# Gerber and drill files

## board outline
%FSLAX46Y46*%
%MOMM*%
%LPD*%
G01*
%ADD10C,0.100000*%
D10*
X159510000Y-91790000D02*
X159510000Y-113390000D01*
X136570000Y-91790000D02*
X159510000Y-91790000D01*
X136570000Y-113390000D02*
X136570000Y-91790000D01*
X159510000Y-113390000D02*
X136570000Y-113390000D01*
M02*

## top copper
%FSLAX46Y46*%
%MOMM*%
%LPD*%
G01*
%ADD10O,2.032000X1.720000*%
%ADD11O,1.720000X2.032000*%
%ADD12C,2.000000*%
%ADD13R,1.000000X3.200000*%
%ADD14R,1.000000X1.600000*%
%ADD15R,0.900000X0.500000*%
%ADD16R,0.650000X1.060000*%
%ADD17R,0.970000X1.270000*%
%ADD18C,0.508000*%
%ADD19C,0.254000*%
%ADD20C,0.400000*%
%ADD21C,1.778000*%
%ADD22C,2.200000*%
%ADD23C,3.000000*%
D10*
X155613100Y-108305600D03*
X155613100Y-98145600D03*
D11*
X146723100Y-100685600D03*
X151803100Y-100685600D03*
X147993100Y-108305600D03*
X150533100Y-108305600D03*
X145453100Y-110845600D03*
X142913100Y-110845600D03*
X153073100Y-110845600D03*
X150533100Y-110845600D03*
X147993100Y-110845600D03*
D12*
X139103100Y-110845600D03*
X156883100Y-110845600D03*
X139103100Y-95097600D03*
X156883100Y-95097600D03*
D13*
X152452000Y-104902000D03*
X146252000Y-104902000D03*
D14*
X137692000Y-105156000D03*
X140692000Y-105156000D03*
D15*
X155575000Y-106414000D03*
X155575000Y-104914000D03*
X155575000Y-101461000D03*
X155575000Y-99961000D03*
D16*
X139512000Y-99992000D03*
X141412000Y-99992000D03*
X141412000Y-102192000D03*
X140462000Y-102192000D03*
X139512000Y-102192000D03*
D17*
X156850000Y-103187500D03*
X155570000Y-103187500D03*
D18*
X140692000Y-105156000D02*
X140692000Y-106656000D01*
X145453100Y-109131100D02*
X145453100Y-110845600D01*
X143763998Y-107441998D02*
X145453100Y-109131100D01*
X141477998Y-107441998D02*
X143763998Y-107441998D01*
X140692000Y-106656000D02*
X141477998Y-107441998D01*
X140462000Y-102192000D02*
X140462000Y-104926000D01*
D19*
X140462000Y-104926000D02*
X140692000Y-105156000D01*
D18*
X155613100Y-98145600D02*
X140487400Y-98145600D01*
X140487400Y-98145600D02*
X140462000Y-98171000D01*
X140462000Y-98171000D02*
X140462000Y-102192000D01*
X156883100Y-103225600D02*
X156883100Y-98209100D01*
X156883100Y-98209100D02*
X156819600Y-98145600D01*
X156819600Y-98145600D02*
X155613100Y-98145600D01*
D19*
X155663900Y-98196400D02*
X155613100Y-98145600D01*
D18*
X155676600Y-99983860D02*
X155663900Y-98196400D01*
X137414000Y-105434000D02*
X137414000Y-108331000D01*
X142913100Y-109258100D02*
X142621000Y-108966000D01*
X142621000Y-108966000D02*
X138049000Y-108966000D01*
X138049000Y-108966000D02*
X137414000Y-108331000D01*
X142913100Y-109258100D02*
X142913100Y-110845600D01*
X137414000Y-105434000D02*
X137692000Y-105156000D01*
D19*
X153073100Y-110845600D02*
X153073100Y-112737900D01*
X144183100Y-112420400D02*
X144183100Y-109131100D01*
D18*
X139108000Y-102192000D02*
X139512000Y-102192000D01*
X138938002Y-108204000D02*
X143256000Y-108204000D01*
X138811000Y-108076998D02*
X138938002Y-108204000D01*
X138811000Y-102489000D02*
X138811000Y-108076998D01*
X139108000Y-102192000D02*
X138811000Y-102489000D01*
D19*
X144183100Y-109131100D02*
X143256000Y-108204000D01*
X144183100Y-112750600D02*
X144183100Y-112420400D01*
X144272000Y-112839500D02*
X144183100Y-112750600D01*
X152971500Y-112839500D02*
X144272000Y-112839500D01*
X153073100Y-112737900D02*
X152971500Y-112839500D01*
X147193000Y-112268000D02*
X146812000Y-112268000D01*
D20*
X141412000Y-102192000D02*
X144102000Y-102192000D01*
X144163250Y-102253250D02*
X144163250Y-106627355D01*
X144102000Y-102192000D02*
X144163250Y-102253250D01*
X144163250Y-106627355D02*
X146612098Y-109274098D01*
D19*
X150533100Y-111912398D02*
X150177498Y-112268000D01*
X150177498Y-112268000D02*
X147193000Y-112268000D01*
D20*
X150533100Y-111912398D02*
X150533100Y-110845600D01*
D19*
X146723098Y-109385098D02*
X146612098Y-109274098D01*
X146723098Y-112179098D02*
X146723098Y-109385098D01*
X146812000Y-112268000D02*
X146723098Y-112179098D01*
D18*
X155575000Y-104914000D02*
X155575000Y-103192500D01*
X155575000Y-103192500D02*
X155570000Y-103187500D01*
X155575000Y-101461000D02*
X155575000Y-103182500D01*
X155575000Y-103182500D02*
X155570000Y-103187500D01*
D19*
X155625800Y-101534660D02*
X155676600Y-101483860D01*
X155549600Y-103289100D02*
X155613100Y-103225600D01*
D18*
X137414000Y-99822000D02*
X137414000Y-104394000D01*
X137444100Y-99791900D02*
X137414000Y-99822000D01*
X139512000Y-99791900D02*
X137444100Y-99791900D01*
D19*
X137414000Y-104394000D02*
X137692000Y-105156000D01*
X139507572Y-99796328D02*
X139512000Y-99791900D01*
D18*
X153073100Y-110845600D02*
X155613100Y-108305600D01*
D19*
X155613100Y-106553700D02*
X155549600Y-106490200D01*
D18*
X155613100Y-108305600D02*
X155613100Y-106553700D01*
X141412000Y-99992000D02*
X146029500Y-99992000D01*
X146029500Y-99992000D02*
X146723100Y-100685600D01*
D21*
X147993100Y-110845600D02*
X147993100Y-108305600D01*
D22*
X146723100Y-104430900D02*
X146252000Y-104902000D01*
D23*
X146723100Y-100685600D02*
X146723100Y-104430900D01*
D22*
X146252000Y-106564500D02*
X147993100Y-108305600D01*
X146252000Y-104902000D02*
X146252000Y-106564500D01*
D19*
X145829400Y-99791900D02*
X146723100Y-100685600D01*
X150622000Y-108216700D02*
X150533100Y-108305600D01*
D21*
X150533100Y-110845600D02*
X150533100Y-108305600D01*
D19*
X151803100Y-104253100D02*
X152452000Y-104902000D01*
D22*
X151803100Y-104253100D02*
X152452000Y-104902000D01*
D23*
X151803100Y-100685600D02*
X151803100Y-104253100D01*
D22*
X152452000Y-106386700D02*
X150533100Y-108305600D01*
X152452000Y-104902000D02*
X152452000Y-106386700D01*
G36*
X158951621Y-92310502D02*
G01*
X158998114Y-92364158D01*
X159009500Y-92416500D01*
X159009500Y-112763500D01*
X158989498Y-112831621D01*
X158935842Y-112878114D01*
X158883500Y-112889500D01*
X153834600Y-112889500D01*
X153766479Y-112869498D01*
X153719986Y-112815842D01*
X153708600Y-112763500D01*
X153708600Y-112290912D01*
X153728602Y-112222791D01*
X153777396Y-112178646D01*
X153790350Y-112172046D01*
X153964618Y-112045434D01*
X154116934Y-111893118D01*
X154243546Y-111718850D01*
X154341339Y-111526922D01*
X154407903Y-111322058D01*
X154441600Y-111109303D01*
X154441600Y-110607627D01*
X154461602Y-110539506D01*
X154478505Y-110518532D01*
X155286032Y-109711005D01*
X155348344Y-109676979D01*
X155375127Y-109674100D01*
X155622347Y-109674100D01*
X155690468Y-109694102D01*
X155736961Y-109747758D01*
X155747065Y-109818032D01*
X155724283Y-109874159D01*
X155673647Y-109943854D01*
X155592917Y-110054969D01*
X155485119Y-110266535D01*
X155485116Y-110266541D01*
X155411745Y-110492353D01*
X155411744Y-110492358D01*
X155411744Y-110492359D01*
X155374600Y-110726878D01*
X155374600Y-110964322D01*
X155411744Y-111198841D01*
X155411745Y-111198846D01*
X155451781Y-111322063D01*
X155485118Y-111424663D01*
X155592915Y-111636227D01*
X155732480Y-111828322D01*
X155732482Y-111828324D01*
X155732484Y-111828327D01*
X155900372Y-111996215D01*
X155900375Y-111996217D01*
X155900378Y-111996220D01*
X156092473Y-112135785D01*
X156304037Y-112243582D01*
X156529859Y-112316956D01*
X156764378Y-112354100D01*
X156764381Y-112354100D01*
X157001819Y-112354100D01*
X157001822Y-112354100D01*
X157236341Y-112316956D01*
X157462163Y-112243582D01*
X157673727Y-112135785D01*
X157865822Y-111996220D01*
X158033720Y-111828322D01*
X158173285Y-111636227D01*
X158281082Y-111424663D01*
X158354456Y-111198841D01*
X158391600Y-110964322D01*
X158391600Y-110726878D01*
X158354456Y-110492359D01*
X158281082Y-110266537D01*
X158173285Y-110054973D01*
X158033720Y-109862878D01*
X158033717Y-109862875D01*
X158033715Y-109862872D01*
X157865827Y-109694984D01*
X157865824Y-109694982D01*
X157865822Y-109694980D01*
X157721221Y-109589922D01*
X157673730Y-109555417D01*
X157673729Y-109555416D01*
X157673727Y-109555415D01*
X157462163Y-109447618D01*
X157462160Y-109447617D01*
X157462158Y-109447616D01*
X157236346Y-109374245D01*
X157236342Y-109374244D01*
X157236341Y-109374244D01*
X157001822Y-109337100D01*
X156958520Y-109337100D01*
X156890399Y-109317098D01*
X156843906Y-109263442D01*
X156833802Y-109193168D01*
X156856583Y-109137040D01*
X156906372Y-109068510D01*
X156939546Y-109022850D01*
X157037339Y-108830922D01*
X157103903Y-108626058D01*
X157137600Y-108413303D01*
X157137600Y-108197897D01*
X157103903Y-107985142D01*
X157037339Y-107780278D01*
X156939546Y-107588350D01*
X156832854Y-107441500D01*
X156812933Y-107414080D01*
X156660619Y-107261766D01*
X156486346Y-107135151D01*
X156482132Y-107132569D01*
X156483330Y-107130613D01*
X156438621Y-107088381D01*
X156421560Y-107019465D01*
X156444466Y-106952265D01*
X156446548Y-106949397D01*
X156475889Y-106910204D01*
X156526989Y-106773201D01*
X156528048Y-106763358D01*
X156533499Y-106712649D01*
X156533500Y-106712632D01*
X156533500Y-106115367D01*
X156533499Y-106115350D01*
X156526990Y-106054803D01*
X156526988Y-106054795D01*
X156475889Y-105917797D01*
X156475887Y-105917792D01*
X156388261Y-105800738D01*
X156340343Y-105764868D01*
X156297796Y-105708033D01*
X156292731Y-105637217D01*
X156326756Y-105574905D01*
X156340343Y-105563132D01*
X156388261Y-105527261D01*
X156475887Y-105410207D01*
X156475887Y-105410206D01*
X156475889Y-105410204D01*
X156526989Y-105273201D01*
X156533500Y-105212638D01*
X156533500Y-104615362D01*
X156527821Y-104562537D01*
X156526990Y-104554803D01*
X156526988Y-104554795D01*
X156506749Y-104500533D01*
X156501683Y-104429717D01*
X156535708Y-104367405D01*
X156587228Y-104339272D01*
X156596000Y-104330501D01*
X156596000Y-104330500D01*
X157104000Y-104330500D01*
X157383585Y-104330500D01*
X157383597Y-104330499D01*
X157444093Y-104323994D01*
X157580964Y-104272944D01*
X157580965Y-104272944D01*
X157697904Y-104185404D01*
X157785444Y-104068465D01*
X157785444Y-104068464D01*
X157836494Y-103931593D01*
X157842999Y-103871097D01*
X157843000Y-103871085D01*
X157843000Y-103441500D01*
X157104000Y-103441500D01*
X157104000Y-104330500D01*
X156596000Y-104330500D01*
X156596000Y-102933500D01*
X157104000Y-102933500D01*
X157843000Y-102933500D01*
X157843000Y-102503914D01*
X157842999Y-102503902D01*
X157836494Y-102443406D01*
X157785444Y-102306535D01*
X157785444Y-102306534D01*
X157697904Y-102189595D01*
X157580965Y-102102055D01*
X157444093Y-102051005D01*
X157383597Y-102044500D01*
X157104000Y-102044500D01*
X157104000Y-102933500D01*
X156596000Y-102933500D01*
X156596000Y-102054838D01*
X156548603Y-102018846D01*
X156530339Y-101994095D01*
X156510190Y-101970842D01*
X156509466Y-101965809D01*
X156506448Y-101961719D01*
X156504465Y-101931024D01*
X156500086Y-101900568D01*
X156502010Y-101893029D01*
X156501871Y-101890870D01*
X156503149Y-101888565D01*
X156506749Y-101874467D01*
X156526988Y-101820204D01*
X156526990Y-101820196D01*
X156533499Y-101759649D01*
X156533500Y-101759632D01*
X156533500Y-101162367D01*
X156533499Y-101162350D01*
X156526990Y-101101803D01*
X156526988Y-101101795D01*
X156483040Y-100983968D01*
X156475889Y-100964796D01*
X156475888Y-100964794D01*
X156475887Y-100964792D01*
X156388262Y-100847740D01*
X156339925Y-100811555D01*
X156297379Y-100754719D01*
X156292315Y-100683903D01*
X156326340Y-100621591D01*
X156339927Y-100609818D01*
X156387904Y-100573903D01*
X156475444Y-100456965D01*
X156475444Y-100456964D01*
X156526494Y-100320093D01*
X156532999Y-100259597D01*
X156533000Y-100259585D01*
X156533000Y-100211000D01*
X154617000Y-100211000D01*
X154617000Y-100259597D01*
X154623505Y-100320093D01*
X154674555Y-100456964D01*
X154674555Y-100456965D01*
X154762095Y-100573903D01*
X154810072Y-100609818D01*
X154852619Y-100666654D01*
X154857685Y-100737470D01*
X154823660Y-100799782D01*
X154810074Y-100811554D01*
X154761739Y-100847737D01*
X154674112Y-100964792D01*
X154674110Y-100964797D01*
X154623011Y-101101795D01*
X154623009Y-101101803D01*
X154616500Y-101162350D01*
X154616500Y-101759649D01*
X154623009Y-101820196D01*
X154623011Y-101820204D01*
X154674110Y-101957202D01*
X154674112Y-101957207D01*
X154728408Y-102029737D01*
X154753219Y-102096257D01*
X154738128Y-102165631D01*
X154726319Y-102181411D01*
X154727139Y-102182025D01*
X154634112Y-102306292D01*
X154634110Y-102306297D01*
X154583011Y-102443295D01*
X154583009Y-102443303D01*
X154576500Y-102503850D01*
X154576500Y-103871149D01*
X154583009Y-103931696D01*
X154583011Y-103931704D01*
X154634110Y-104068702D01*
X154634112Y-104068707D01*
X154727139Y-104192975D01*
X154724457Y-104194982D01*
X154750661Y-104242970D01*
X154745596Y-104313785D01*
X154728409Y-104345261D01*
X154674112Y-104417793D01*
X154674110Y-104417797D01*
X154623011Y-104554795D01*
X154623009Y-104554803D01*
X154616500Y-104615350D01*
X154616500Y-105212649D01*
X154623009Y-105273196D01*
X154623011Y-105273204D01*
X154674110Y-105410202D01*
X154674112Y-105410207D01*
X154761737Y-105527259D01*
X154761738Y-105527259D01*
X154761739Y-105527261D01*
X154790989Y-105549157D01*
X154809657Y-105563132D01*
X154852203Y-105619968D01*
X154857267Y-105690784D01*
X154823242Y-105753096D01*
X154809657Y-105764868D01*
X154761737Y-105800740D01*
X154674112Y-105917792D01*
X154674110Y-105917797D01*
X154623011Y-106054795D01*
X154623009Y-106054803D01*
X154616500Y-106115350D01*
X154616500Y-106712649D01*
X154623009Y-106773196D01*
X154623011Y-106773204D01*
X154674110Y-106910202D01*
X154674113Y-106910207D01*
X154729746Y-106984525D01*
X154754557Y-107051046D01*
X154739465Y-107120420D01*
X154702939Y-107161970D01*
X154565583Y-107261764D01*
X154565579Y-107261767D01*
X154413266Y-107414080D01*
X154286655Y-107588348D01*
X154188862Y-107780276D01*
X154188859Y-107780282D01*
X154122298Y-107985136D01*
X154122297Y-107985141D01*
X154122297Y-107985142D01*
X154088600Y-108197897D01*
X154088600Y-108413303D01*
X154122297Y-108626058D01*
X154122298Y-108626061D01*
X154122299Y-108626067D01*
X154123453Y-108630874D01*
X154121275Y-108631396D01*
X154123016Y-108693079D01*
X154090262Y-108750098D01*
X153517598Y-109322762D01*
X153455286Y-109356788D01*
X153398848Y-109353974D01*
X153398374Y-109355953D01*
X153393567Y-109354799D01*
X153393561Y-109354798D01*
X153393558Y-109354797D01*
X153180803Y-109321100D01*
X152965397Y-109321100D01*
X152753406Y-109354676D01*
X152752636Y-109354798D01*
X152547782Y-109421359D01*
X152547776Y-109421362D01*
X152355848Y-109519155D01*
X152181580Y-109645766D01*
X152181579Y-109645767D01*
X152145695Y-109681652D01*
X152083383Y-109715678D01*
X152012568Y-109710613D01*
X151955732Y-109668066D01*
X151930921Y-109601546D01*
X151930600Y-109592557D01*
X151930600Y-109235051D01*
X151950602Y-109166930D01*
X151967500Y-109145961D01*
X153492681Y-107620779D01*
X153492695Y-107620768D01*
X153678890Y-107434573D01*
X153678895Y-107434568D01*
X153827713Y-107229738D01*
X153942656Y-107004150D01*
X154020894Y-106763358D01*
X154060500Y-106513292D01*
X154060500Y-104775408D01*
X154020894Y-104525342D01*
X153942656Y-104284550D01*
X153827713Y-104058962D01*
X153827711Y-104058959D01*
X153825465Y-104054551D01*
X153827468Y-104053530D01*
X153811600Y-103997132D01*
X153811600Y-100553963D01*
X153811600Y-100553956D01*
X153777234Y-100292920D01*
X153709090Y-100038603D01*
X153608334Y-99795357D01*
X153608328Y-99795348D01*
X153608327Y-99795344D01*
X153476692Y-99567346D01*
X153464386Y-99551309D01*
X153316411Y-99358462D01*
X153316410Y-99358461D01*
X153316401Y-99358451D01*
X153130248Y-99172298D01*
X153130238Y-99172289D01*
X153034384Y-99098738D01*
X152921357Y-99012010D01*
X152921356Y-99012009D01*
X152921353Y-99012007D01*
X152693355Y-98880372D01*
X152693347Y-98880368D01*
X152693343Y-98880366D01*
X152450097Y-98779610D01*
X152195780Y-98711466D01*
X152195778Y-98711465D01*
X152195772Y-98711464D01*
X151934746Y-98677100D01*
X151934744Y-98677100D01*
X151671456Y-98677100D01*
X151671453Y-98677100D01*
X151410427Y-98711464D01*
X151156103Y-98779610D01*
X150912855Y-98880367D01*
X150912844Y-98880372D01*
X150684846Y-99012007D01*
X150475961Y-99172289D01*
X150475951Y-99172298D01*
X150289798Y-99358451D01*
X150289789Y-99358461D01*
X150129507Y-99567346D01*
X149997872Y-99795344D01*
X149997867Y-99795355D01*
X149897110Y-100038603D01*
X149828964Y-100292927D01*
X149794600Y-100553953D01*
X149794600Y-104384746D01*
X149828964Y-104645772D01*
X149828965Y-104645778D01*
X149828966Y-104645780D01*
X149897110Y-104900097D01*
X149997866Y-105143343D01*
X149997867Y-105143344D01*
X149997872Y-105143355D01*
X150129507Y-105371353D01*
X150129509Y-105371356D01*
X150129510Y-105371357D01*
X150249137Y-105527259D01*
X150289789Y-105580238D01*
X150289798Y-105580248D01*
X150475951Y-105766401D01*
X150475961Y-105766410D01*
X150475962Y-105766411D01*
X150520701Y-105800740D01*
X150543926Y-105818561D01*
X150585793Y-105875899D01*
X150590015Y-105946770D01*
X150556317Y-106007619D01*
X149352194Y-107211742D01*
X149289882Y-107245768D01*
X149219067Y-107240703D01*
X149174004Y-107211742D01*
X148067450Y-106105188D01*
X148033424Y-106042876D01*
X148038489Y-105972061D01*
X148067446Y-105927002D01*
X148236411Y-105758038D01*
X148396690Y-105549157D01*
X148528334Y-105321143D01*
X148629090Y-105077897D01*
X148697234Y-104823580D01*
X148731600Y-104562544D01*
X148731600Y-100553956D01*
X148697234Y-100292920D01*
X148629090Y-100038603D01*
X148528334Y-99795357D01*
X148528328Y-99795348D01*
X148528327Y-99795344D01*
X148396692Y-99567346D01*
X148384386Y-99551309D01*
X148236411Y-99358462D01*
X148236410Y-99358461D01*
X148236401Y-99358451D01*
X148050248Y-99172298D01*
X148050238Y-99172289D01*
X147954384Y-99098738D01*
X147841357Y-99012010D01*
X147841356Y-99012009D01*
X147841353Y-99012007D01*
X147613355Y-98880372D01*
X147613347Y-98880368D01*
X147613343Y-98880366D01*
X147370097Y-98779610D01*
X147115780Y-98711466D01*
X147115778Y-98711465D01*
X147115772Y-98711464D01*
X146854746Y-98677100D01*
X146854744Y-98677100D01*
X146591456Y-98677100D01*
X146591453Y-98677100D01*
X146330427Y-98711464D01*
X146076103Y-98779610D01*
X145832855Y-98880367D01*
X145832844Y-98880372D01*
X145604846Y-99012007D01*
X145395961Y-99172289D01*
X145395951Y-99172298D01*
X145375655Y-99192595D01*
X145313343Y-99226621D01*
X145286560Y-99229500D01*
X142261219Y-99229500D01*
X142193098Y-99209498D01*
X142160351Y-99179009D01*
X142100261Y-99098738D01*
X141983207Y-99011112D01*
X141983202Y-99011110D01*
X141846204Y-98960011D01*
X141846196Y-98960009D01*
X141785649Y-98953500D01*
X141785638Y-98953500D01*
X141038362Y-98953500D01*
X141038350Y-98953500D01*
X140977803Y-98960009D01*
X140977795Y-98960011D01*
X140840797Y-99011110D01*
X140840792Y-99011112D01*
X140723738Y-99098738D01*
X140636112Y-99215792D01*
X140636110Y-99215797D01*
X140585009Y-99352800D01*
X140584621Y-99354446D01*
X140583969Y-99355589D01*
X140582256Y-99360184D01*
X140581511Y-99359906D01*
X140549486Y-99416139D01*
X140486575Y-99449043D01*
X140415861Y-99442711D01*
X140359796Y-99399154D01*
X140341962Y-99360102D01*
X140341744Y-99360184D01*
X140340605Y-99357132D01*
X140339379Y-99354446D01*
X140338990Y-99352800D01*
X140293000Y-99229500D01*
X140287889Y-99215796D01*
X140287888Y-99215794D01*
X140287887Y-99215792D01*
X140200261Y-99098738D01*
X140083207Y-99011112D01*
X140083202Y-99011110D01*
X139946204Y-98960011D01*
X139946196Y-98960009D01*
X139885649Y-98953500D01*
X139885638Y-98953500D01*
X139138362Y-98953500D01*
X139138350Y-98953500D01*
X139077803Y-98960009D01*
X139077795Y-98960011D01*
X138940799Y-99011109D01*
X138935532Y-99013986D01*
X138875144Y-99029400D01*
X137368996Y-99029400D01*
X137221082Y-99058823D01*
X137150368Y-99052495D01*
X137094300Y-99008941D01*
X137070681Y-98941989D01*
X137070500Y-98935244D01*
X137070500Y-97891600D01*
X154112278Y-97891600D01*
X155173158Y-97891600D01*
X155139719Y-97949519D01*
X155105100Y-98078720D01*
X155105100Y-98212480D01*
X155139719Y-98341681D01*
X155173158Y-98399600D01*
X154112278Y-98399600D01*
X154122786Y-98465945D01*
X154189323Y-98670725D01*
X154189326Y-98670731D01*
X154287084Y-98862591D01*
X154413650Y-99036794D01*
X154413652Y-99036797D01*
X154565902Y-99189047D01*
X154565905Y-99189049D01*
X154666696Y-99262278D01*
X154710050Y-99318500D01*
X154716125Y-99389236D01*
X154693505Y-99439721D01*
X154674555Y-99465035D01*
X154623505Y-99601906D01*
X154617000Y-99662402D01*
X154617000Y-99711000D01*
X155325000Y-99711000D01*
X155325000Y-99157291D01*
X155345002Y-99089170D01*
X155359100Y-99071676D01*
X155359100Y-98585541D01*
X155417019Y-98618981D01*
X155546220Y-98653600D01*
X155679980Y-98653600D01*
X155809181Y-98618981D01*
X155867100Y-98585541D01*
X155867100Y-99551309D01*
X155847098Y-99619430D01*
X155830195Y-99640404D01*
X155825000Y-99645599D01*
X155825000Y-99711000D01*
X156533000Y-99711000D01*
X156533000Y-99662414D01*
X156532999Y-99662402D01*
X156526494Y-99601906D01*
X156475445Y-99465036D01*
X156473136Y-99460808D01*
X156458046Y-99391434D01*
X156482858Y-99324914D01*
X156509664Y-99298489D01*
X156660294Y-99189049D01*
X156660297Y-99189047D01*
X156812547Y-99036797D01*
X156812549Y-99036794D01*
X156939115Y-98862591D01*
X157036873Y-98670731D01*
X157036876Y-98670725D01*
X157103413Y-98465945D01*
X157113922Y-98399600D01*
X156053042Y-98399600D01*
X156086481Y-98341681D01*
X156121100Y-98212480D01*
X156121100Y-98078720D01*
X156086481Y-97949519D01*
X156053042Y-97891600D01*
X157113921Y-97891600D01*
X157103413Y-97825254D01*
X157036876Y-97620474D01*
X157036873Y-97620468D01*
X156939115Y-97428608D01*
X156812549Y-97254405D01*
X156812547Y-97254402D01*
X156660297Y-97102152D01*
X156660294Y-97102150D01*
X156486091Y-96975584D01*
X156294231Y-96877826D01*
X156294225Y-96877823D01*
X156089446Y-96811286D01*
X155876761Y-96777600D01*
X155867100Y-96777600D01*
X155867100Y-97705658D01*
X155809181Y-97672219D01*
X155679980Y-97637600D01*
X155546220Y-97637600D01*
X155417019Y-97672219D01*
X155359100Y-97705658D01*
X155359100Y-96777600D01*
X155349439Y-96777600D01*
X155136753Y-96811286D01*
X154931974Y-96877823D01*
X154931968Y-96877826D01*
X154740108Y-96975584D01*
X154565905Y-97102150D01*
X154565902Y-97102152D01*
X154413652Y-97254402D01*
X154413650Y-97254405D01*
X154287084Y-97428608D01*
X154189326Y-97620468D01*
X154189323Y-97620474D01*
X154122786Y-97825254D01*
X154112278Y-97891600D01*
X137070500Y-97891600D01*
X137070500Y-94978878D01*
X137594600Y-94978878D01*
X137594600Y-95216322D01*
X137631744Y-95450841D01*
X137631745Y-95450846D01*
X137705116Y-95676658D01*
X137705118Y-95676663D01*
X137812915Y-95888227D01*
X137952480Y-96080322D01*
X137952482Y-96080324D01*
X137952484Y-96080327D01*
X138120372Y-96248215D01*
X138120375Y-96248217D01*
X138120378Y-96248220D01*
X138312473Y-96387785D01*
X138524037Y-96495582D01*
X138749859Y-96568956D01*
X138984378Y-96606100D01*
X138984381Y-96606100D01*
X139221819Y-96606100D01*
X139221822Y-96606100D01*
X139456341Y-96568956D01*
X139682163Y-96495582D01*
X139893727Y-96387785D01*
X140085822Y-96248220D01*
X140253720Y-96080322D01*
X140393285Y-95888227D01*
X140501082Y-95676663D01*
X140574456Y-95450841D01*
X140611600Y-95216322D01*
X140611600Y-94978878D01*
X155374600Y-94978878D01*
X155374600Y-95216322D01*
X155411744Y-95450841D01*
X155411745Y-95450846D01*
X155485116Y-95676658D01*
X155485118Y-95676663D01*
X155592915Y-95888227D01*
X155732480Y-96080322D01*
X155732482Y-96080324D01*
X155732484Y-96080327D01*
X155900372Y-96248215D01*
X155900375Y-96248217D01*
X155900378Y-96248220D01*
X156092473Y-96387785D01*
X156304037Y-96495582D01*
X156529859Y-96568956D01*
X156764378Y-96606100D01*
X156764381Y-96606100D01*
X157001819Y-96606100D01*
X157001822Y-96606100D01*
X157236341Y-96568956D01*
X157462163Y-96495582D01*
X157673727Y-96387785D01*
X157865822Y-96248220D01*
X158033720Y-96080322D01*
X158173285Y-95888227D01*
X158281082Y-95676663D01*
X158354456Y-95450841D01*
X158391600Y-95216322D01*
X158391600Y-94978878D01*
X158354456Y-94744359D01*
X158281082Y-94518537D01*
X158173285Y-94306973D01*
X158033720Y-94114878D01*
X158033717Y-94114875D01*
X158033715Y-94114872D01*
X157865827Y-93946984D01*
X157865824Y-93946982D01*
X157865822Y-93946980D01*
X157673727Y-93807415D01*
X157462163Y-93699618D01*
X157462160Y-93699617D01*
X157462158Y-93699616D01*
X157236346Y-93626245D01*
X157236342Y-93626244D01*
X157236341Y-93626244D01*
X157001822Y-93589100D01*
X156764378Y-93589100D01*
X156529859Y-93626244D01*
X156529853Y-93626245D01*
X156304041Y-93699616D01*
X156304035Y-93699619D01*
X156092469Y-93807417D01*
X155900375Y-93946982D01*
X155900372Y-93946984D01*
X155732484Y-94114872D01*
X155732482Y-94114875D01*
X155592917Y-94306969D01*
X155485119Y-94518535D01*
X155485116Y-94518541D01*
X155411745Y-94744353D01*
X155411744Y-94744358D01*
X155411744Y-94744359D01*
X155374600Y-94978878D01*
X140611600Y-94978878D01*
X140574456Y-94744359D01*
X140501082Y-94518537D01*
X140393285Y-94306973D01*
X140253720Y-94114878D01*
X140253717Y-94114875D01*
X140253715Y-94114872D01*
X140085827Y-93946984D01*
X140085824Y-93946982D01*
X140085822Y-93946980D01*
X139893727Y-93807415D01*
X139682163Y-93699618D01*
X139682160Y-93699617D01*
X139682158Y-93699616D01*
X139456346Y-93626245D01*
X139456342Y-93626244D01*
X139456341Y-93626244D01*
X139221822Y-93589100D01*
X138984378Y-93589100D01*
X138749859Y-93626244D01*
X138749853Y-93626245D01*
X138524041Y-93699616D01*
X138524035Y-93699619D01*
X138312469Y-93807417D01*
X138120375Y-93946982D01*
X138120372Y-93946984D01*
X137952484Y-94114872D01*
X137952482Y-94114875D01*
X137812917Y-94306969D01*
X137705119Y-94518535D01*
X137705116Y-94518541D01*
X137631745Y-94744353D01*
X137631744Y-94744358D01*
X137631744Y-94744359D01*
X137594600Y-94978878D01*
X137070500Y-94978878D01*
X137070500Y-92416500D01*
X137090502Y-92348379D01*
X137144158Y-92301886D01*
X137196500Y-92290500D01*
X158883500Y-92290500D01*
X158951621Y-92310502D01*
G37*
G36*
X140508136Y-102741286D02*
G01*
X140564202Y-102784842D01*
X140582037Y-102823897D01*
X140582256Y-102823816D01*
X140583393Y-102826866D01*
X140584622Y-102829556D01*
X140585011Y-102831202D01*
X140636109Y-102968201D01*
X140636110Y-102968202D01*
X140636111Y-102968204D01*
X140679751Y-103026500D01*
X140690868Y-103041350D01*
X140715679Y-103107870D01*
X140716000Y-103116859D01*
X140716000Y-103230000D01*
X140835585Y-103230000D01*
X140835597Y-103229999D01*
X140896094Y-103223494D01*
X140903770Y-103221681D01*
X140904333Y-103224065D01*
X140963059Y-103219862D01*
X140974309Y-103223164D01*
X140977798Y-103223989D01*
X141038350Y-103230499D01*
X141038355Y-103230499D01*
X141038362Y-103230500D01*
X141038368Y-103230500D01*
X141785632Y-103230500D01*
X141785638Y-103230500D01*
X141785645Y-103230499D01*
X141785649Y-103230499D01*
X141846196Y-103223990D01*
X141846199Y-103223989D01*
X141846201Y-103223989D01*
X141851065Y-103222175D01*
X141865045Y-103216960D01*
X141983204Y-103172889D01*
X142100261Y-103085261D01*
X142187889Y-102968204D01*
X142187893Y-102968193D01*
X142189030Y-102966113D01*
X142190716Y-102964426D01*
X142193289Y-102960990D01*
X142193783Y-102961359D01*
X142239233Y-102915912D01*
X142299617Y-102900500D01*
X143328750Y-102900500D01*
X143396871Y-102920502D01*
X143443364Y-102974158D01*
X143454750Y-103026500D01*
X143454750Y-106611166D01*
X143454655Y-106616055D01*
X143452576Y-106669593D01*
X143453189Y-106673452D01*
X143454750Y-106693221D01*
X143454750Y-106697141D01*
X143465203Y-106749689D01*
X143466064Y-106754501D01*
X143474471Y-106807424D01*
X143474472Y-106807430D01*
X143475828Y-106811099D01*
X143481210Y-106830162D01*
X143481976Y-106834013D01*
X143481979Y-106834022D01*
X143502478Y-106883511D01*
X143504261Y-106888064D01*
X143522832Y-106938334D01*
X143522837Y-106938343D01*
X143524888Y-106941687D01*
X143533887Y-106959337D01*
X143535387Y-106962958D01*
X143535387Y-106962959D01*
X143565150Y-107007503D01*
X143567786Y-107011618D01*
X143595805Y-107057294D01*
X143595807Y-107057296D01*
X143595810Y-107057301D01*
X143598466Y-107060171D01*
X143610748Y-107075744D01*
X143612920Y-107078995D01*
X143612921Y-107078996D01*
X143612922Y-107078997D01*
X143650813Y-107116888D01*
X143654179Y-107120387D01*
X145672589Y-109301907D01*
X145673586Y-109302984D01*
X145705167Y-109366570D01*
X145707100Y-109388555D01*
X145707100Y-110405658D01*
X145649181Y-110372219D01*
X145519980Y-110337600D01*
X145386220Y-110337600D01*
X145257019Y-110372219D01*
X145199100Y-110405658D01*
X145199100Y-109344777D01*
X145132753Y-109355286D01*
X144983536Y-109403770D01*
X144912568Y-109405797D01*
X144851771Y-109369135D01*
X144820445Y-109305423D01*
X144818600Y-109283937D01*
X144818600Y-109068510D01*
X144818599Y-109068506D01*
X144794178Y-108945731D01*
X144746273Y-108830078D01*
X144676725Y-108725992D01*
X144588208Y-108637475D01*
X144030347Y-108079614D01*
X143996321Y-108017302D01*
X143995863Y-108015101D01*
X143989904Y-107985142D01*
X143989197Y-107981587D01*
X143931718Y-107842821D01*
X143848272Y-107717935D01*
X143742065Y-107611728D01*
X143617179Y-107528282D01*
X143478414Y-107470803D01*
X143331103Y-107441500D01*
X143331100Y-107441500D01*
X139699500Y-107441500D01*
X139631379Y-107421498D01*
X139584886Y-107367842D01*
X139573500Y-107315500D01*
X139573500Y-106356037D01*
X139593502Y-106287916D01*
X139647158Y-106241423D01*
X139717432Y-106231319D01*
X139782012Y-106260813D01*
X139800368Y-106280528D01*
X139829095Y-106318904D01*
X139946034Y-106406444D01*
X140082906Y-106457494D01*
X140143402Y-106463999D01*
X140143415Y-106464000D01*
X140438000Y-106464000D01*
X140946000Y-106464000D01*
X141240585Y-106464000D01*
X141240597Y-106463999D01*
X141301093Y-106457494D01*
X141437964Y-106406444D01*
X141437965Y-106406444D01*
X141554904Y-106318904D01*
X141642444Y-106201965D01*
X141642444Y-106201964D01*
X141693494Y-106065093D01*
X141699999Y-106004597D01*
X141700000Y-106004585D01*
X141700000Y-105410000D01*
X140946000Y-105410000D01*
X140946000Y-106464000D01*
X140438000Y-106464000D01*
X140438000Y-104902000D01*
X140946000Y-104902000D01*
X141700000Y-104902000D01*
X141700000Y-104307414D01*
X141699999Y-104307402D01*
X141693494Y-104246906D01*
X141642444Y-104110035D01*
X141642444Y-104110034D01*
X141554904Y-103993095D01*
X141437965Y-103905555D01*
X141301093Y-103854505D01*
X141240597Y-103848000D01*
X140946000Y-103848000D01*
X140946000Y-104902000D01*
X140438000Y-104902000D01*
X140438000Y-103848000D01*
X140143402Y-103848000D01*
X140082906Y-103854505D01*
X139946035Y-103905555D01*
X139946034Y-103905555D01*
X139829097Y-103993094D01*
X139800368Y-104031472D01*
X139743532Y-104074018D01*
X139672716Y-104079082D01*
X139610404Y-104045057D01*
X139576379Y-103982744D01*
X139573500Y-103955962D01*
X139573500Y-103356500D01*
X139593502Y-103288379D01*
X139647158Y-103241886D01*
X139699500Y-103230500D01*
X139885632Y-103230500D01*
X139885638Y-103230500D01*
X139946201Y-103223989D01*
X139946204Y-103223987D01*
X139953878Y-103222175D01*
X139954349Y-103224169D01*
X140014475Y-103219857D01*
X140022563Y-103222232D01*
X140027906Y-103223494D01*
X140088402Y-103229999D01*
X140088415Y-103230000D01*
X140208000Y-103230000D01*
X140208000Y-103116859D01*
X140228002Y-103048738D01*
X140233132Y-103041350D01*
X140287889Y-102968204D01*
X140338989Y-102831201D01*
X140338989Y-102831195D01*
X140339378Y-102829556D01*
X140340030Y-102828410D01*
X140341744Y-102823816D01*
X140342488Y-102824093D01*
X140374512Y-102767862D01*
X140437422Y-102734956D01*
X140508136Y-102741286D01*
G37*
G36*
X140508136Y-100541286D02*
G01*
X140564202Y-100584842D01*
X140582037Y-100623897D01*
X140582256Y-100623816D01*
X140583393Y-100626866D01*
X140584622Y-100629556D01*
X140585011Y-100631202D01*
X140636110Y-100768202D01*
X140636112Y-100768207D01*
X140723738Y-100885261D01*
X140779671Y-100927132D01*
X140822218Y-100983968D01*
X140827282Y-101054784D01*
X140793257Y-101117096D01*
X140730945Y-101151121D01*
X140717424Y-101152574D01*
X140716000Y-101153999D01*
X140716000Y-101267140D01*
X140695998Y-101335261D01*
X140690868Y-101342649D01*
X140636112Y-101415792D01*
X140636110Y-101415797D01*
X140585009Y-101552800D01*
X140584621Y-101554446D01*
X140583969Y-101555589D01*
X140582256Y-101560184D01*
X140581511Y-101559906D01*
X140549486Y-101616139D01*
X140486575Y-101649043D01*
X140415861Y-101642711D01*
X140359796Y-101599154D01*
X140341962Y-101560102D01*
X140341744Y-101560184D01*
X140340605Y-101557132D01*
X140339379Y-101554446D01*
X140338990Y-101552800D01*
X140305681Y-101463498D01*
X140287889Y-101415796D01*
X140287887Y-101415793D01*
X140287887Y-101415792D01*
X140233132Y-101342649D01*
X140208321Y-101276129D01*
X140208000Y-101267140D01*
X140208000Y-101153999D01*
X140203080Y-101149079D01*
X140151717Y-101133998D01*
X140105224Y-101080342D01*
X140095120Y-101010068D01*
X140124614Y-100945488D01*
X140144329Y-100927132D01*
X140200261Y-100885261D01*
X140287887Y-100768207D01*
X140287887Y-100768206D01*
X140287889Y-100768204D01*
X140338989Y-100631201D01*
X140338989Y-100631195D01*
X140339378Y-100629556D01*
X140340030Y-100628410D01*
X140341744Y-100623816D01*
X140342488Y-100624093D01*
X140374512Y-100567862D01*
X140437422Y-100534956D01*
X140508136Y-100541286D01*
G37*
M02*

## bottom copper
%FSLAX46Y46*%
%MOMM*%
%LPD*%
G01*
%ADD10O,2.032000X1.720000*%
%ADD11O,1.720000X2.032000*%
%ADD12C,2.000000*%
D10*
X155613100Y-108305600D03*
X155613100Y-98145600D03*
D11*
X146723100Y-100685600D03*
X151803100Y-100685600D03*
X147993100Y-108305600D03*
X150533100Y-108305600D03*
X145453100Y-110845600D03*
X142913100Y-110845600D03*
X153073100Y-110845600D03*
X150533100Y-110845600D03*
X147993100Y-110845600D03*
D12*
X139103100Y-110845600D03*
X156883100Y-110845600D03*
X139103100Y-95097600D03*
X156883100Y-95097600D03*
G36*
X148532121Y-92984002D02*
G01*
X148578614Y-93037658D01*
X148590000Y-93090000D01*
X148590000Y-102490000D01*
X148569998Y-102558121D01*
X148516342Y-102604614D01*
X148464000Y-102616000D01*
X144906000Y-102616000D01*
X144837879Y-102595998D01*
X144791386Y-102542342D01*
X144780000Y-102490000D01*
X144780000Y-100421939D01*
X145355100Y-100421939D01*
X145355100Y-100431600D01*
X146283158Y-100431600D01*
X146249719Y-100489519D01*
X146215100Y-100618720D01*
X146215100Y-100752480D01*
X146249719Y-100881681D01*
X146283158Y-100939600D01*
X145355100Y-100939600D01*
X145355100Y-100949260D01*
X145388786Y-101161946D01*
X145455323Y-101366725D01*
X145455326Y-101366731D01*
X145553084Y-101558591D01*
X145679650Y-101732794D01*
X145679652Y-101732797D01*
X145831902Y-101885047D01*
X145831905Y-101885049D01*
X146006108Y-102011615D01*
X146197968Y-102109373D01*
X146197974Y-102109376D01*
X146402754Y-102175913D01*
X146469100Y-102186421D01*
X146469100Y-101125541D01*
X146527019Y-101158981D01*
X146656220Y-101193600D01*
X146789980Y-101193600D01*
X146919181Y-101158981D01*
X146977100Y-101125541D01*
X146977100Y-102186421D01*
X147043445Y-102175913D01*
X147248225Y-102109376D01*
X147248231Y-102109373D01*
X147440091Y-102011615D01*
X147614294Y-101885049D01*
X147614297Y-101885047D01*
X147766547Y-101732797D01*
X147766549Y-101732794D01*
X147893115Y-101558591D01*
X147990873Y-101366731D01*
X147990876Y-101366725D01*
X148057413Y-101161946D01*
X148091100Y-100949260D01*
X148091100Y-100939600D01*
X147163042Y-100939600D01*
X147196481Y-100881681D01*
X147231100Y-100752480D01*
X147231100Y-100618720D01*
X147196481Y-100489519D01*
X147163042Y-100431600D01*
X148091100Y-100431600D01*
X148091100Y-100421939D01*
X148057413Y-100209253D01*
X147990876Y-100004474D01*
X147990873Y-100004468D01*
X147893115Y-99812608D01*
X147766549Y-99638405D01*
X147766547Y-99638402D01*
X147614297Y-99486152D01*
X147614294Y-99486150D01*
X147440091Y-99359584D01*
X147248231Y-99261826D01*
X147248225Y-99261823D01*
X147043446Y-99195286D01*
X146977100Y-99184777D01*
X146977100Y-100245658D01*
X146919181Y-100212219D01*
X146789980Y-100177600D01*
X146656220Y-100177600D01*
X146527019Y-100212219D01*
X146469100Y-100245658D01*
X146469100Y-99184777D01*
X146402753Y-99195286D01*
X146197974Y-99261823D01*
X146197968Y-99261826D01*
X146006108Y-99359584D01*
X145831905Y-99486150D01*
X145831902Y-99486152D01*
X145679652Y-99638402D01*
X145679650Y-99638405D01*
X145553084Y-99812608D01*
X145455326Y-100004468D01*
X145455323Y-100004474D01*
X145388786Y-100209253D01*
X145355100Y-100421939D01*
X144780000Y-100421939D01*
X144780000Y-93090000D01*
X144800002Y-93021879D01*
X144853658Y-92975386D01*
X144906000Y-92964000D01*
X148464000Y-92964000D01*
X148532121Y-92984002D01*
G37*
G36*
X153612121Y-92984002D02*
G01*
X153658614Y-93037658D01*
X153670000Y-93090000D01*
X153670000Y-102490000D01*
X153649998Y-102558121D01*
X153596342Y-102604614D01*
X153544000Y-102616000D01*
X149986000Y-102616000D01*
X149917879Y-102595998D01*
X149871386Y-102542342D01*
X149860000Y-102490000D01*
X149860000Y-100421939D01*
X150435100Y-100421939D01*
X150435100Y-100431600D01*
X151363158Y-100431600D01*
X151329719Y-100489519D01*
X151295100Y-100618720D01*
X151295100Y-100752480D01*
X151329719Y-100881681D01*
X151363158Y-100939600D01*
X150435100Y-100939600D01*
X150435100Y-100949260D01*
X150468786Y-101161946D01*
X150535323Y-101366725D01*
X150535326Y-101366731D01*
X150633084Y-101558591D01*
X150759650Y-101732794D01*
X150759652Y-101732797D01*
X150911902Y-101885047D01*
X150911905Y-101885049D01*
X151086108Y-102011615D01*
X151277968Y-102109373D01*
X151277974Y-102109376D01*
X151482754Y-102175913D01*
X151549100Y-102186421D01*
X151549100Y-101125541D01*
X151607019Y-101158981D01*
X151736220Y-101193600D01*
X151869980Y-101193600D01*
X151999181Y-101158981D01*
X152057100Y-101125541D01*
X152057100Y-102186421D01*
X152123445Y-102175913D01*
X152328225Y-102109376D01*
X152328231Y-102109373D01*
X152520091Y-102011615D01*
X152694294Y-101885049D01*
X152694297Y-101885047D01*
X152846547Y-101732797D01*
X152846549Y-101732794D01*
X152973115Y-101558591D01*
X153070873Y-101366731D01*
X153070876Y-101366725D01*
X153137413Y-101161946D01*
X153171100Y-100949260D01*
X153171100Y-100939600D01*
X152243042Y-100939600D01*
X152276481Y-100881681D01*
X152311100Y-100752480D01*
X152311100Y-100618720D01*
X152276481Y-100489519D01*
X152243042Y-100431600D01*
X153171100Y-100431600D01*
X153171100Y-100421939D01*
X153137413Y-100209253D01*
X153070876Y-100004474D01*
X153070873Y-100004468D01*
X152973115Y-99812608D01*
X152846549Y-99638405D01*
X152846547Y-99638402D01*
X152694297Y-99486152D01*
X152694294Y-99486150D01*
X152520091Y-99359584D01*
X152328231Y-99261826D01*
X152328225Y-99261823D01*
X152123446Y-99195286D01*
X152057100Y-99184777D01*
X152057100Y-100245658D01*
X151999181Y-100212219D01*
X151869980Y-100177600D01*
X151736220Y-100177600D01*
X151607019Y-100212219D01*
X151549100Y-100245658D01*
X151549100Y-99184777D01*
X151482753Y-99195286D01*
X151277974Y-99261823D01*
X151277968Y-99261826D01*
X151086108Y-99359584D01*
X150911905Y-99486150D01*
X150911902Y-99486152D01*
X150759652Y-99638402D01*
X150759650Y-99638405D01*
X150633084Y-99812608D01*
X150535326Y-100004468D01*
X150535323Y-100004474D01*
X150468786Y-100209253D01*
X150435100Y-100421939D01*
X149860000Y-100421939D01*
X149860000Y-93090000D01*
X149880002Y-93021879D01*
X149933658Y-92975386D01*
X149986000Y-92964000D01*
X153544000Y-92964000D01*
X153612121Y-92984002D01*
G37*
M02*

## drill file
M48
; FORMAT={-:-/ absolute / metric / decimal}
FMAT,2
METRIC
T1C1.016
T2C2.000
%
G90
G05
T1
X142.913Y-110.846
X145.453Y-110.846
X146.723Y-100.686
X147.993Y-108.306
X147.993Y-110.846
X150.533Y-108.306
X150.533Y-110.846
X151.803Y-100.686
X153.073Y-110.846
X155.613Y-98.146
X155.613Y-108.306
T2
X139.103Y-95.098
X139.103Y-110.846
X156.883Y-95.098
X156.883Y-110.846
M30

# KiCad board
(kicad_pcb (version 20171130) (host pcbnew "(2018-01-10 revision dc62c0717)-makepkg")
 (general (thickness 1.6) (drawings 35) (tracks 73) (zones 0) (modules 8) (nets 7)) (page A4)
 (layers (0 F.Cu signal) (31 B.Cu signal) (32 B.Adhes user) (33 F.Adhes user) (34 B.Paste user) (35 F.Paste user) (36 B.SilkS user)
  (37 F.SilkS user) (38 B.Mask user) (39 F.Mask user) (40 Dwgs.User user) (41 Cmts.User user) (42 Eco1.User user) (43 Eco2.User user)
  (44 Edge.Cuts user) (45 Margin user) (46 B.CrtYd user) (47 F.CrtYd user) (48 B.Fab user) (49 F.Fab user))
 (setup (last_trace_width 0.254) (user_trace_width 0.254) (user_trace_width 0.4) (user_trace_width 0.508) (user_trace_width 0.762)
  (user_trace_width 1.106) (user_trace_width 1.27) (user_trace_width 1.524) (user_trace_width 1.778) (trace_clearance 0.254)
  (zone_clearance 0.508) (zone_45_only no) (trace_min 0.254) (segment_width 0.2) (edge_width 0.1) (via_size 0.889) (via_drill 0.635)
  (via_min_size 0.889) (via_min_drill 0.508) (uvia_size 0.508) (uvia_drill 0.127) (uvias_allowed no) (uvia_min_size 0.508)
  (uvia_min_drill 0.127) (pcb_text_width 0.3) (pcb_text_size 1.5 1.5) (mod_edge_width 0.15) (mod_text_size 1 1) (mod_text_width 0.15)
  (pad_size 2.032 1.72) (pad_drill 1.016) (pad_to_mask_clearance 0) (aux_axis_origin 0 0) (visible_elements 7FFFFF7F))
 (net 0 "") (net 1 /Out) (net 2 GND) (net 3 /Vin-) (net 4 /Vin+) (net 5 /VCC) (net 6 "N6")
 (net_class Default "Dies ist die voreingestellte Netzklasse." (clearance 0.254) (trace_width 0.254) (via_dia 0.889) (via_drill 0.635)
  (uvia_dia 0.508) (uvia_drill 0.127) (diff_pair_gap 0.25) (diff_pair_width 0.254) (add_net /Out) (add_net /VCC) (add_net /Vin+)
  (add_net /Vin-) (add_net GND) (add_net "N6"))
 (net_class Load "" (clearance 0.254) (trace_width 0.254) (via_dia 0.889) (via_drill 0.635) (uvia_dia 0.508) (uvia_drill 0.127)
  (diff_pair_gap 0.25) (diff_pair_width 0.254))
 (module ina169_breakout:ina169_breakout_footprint (layer F.Cu) (at 147.9931 103.2256)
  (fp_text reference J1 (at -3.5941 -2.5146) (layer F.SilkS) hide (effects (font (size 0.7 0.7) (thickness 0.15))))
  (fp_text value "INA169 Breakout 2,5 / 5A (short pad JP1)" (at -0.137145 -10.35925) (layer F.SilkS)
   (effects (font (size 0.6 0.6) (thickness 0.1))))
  (pad 5 thru_hole oval (at 7.62 5.08) (size 2.032 1.72) (drill 1.016) (layers *.Cu *.Mask F.SilkS) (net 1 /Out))
  (pad 2 thru_hole oval (at 7.62 -5.08) (size 2.032 1.72) (drill 1.016) (layers *.Cu *.Mask F.SilkS) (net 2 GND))
  (pad 3 thru_hole oval (at -1.27 -2.54) (size 1.72 2.032) (drill 1.016) (layers *.Cu *.Mask F.SilkS) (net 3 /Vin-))
  (pad 4 thru_hole oval (at 3.81 -2.54) (size 1.72 2.032) (drill 1.016) (layers *.Cu *.Mask F.SilkS) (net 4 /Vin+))
  (pad 3 thru_hole oval (at 0 5.08) (size 1.72 2.032) (drill 1.016) (layers *.Cu *.Mask F.SilkS) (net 3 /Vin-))
  (pad 4 thru_hole oval (at 2.54 5.08) (size 1.72 2.032) (drill 1.016) (layers *.Cu *.Mask F.SilkS) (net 4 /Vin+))
  (pad 2 thru_hole oval (at -2.54 7.62) (size 1.72 2.032) (drill 1.016) (layers *.Cu *.Mask F.SilkS) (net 2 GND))
  (pad 1 thru_hole oval (at -5.08 7.62) (size 1.72 2.032) (drill 1.016) (layers *.Cu *.Mask F.SilkS) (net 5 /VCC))
  (pad 5 thru_hole oval (at 5.08 7.62) (size 1.72 2.032) (drill 1.016) (layers *.Cu *.Mask F.SilkS) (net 1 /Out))
  (pad 4 thru_hole oval (at 2.54 7.62) (size 1.72 2.032) (drill 1.016) (layers *.Cu *.Mask F.SilkS) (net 4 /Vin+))
  (pad 3 thru_hole oval (at 0 7.62) (size 1.72 2.032) (drill 1.016) (layers *.Cu *.Mask F.SilkS) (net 3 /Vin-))
  (pad "" thru_hole circle (at -8.89 7.62) (size 2 2) (drill 2) (layers *.Cu *.Mask F.SilkS))
  (pad "" thru_hole circle (at 8.89 7.62) (size 2 2) (drill 2) (layers *.Cu *.Mask F.SilkS))
  (pad "" thru_hole circle (at -8.89 -8.128) (size 2 2) (drill 2) (layers *.Cu *.Mask F.SilkS))
  (pad "" thru_hole circle (at 8.89 -8.128) (size 2 2) (drill 2) (layers *.Cu *.Mask F.SilkS)))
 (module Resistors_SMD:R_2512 (layer F.Cu) (at 149.352 104.902 180)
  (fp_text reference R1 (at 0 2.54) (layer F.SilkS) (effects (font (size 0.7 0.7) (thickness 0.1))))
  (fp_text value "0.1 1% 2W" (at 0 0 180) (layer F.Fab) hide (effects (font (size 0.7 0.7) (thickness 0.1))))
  (pad 1 smd rect (at -3.1 0 180) (size 1 3.2) (layers F.Cu F.Paste F.Mask) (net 4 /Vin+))
  (pad 2 smd rect (at 3.1 0 180) (size 1 3.2) (layers F.Cu F.Paste F.Mask) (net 3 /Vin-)))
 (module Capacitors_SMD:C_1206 (layer F.Cu) (at 139.192 105.156)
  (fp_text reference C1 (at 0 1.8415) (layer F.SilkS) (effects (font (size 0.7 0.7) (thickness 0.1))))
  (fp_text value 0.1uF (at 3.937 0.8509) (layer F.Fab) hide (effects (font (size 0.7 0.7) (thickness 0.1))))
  (pad 1 smd rect (at -1.5 0) (size 1 1.6) (layers F.Cu F.Paste F.Mask) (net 5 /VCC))
  (pad 2 smd rect (at 1.5 0) (size 1 1.6) (layers F.Cu F.Paste F.Mask) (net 2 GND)))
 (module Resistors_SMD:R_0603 (layer F.Cu) (at 155.575 105.664 90)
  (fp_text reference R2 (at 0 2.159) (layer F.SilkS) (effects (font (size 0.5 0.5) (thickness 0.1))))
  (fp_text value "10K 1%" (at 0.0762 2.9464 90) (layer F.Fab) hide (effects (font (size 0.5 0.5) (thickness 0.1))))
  (pad 1 smd rect (at -0.75 0 90) (size 0.5 0.9) (layers F.Cu F.Paste F.Mask) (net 1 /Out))
  (pad 2 smd rect (at 0.75 0 90) (size 0.5 0.9) (layers F.Cu F.Paste F.Mask) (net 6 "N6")))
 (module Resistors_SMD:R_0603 (layer F.Cu) (at 155.575 100.711 90)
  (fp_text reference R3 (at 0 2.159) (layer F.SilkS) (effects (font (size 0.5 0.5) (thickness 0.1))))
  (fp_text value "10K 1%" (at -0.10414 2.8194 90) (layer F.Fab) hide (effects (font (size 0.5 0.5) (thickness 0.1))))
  (pad 1 smd rect (at -0.75 0 90) (size 0.5 0.9) (layers F.Cu F.Paste F.Mask) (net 6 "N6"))
  (pad 2 smd rect (at 0.75 0 90) (size 0.5 0.9) (layers F.Cu F.Paste F.Mask) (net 2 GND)))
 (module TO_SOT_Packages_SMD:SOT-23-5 (layer F.Cu) (at 140.462 101.092 90)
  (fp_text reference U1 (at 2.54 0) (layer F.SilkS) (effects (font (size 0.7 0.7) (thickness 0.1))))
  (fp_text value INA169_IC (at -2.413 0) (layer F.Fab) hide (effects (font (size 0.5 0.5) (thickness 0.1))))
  (pad 5 smd rect (at 1.1 -0.95 90) (size 1.06 0.65) (layers F.Cu F.Paste F.Mask) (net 5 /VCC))
  (pad 4 smd rect (at 1.1 0.95 90) (size 1.06 0.65) (layers F.Cu F.Paste F.Mask) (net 3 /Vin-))
  (pad 3 smd rect (at -1.1 0.95 90) (size 1.06 0.65) (layers F.Cu F.Paste F.Mask) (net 4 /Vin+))
  (pad 2 smd rect (at -1.1 0 90) (size 1.06 0.65) (layers F.Cu F.Paste F.Mask) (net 2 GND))
  (pad 1 smd rect (at -1.1 -0.95 90) (size 1.06 0.65) (layers F.Cu F.Paste F.Mask) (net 1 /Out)))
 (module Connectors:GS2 (layer F.Cu) (at 156.21 103.1875 90)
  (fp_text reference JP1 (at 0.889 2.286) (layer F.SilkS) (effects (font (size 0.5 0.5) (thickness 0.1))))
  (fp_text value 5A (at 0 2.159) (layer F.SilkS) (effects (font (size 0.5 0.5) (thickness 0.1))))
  (pad 2 smd rect (at 0 0.64 90) (size 1.27 0.97) (layers F.Cu F.Paste F.Mask) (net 2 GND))
  (pad 1 smd rect (at 0 -0.64 90) (size 1.27 0.97) (layers F.Cu F.Paste F.Mask) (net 6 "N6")))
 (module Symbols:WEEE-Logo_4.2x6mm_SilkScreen (layer F.Cu) (at 143.129 106.172)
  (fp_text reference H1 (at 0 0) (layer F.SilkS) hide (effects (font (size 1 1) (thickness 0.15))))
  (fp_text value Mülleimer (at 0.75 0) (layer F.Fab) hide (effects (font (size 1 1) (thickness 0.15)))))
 (gr_line (start 159.51 91.79) (end 159.51 113.39) (angle 90) (layer Edge.Cuts) (width 0.1))
 (gr_line (start 136.57 91.79) (end 159.51 91.79) (angle 90) (layer Edge.Cuts) (width 0.1))
 (gr_line (start 136.57 113.39) (end 136.57 91.79) (angle 90) (layer Edge.Cuts) (width 0.1))
 (gr_line (start 159.51 113.39) (end 136.57 113.39) (angle 90) (layer Edge.Cuts) (width 0.1))
 (segment (start 140.692 105.156) (end 140.692 106.656) (width 0.508) (layer F.Cu) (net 2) (status 400000))
 (segment (start 145.4531 109.1311) (end 145.4531 110.8456) (width 0.508) (layer F.Cu) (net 2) (status 800000))
 (segment (start 143.763998 107.441998) (end 145.4531 109.1311) (width 0.508) (layer F.Cu) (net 2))
 (segment (start 141.477998 107.441998) (end 143.763998 107.441998) (width 0.508) (layer F.Cu) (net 2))
 (segment (start 140.692 106.656) (end 141.477998 107.441998) (width 0.508) (layer F.Cu) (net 2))
 (segment (start 140.462 102.192) (end 140.462 104.926) (width 0.508) (layer F.Cu) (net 2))
 (segment (start 140.462 104.926) (end 140.692 105.156) (width 0.254) (layer F.Cu) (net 2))
 (segment (start 155.6131 98.1456) (end 140.4874 98.1456) (width 0.508) (layer F.Cu) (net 2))
 (segment (start 140.4874 98.1456) (end 140.462 98.171) (width 0.508) (layer F.Cu) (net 2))
 (segment (start 140.462 98.171) (end 140.462 102.192) (width 0.508) (layer F.Cu) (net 2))
 (segment (start 156.8831 103.2256) (end 156.8831 98.2091) (width 0.508) (layer F.Cu) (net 2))
 (segment (start 156.8831 98.2091) (end 156.8196 98.1456) (width 0.508) (layer F.Cu) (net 2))
 (segment (start 156.8196 98.1456) (end 155.6131 98.1456) (width 0.508) (layer F.Cu) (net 2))
 (segment (start 155.6639 98.1964) (end 155.6131 98.1456) (width 0.254) (layer F.Cu) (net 2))
 (segment (start 155.6766 99.98386) (end 155.6639 98.1964) (width 0.508) (layer F.Cu) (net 2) (status 10))
 (segment (start 137.414 105.434) (end 137.414 108.331) (width 0.508) (layer F.Cu) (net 5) (status 400000))
 (segment (start 142.9131 109.2581) (end 142.621 108.966) (width 0.508) (layer F.Cu) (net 5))
 (segment (start 142.621 108.966) (end 138.049 108.966) (width 0.508) (layer F.Cu) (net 5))
 (segment (start 138.049 108.966) (end 137.414 108.331) (width 0.508) (layer F.Cu) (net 5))
 (segment (start 142.9131 109.2581) (end 142.9131 110.8456) (width 0.508) (layer F.Cu) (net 5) (status 800000))
 (segment (start 137.414 105.434) (end 137.692 105.156) (width 0.508) (layer F.Cu) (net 5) (status C00000))
 (segment (start 153.0731 110.8456) (end 153.0731 112.7379) (width 0.254) (layer F.Cu) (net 1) (status 400000))
 (segment (start 144.1831 112.4204) (end 144.1831 109.1311) (width 0.254) (layer F.Cu) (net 1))
 (segment (start 139.108 102.192) (end 139.512 102.192) (width 0.508) (layer F.Cu) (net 1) (status 800000))
 (segment (start 138.938002 108.204) (end 143.256 108.204) (width 0.508) (layer F.Cu) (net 1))
 (segment (start 138.811 108.076998) (end 138.938002 108.204) (width 0.508) (layer F.Cu) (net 1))
 (segment (start 138.811 102.489) (end 138.811 108.076998) (width 0.508) (layer F.Cu) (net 1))
 (segment (start 139.108 102.192) (end 138.811 102.489) (width 0.508) (layer F.Cu) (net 1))
 (segment (start 144.1831 109.1311) (end 143.256 108.204) (width 0.254) (layer F.Cu) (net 1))
 (segment (start 144.1831 112.7506) (end 144.1831 112.4204) (width 0.254) (layer F.Cu) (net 1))
 (segment (start 144.272 112.8395) (end 144.1831 112.7506) (width 0.254) (layer F.Cu) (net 1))
 (segment (start 152.9715 112.8395) (end 144.272 112.8395) (width 0.254) (layer F.Cu) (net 1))
 (segment (start 153.0731 112.7379) (end 152.9715 112.8395) (width 0.254) (layer F.Cu) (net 1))
 (segment (start 147.193 112.268) (end 146.812 112.268) (width 0.254) (layer F.Cu) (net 4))
 (segment (start 141.412 102.192) (end 144.102 102.192) (width 0.4) (layer F.Cu) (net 4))
 (segment (start 144.16325 102.25325) (end 144.16325 106.627355) (width 0.4) (layer F.Cu) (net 4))
 (segment (start 144.102 102.192) (end 144.16325 102.25325) (width 0.4) (layer F.Cu) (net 4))
 (segment (start 144.16325 106.627355) (end 146.612098 109.274098) (width 0.4) (layer F.Cu) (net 4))
 (segment (start 150.5331 111.912398) (end 150.177498 112.268) (width 0.254) (layer F.Cu) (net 4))
 (segment (start 150.177498 112.268) (end 147.193 112.268) (width 0.254) (layer F.Cu) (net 4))
 (segment (start 150.5331 111.912398) (end 150.5331 110.8456) (width 0.4) (layer F.Cu) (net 4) (status 800000))
 (segment (start 146.723098 109.385098) (end 146.612098 109.274098) (width 0.254) (layer F.Cu) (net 4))
 (segment (start 146.723098 112.179098) (end 146.723098 109.385098) (width 0.254) (layer F.Cu) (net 4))
 (segment (start 146.812 112.268) (end 146.723098 112.179098) (width 0.254) (layer F.Cu) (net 4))
 (segment (start 155.575 104.914) (end 155.575 103.1925) (width 0.508) (layer F.Cu) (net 6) (status C00000))
 (segment (start 155.575 103.1925) (end 155.57 103.1875) (width 0.508) (layer F.Cu) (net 6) (status C00000))
 (segment (start 155.575 101.461) (end 155.575 103.1825) (width 0.508) (layer F.Cu) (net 6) (status C00000))
 (segment (start 155.575 103.1825) (end 155.57 103.1875) (width 0.508) (layer F.Cu) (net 6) (status C00000))
 (segment (start 155.6258 101.53466) (end 155.6766 101.48386) (width 0.254) (layer F.Cu) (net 6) (status 30))
 (segment (start 155.5496 103.2891) (end 155.6131 103.2256) (width 0.254) (layer F.Cu) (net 6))
 (segment (start 137.414 99.822) (end 137.414 104.394) (width 0.508) (layer F.Cu) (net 5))
 (segment (start 137.4441 99.7919) (end 137.414 99.822) (width 0.508) (layer F.Cu) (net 5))
 (segment (start 139.512 99.7919) (end 137.4441 99.7919) (width 0.508) (layer F.Cu) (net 5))
 (segment (start 137.414 104.394) (end 137.692 105.156) (width 0.254) (layer F.Cu) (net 5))
 (segment (start 139.507572 99.796328) (end 139.512 99.7919) (width 0.254) (layer F.Cu) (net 5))
 (segment (start 153.0731 110.8456) (end 155.6131 108.3056) (width 0.508) (layer F.Cu) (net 1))
 (segment (start 155.6131 106.5537) (end 155.5496 106.4902) (width 0.254) (layer F.Cu) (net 1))
 (segment (start 155.6131 108.3056) (end 155.6131 106.5537) (width 0.508) (layer F.Cu) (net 1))
 (segment (start 141.412 99.992) (end 146.0295 99.992) (width 0.508) (layer F.Cu) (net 3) (status 400000))
 (segment (start 146.0295 99.992) (end 146.7231 100.6856) (width 0.508) (layer F.Cu) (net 3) (status 800000))
 (segment (start 147.9931 110.8456) (end 147.9931 108.3056) (width 1.778) (layer F.Cu) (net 3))
 (segment (start 146.7231 104.4309) (end 146.252 104.902) (width 2.2) (layer F.Cu) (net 3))
 (segment (start 146.7231 100.6856) (end 146.7231 104.4309) (width 3) (layer F.Cu) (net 3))
 (segment (start 146.252 106.5645) (end 147.9931 108.3056) (width 2.2) (layer F.Cu) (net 3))
 (segment (start 146.252 104.902) (end 146.252 106.5645) (width 2.2) (layer F.Cu) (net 3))
 (segment (start 145.8294 99.7919) (end 146.7231 100.6856) (width 0.254) (layer F.Cu) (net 3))
 (segment (start 150.622 108.2167) (end 150.5331 108.3056) (width 0.254) (layer F.Cu) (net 4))
 (segment (start 150.5331 110.8456) (end 150.5331 108.3056) (width 1.778) (layer F.Cu) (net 4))
 (segment (start 151.8031 104.2531) (end 152.452 104.902) (width 0.254) (layer F.Cu) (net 4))
 (segment (start 151.8031 104.2531) (end 152.452 104.902) (width 2.2) (layer F.Cu) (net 4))
 (segment (start 151.8031 100.6856) (end 151.8031 104.2531) (width 3) (layer F.Cu) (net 4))
 (segment (start 152.452 106.3867) (end 150.5331 108.3056) (width 2.2) (layer F.Cu) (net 4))
 (segment (start 152.452 104.902) (end 152.452 106.3867) (width 2.2) (layer F.Cu) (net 4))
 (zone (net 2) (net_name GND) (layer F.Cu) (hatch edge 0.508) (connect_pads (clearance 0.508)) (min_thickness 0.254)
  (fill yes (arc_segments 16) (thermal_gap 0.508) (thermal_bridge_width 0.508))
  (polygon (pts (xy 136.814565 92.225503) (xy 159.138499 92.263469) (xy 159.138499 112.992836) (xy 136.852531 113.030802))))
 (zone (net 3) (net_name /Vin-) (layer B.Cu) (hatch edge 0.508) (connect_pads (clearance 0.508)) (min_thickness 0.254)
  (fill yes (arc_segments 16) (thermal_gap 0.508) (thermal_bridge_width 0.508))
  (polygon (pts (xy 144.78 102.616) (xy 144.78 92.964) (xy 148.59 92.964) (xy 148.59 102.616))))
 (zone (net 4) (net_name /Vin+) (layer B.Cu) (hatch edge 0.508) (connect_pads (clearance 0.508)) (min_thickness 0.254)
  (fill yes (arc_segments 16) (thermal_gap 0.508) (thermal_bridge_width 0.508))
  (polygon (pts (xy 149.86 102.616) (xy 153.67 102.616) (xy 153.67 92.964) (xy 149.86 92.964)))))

